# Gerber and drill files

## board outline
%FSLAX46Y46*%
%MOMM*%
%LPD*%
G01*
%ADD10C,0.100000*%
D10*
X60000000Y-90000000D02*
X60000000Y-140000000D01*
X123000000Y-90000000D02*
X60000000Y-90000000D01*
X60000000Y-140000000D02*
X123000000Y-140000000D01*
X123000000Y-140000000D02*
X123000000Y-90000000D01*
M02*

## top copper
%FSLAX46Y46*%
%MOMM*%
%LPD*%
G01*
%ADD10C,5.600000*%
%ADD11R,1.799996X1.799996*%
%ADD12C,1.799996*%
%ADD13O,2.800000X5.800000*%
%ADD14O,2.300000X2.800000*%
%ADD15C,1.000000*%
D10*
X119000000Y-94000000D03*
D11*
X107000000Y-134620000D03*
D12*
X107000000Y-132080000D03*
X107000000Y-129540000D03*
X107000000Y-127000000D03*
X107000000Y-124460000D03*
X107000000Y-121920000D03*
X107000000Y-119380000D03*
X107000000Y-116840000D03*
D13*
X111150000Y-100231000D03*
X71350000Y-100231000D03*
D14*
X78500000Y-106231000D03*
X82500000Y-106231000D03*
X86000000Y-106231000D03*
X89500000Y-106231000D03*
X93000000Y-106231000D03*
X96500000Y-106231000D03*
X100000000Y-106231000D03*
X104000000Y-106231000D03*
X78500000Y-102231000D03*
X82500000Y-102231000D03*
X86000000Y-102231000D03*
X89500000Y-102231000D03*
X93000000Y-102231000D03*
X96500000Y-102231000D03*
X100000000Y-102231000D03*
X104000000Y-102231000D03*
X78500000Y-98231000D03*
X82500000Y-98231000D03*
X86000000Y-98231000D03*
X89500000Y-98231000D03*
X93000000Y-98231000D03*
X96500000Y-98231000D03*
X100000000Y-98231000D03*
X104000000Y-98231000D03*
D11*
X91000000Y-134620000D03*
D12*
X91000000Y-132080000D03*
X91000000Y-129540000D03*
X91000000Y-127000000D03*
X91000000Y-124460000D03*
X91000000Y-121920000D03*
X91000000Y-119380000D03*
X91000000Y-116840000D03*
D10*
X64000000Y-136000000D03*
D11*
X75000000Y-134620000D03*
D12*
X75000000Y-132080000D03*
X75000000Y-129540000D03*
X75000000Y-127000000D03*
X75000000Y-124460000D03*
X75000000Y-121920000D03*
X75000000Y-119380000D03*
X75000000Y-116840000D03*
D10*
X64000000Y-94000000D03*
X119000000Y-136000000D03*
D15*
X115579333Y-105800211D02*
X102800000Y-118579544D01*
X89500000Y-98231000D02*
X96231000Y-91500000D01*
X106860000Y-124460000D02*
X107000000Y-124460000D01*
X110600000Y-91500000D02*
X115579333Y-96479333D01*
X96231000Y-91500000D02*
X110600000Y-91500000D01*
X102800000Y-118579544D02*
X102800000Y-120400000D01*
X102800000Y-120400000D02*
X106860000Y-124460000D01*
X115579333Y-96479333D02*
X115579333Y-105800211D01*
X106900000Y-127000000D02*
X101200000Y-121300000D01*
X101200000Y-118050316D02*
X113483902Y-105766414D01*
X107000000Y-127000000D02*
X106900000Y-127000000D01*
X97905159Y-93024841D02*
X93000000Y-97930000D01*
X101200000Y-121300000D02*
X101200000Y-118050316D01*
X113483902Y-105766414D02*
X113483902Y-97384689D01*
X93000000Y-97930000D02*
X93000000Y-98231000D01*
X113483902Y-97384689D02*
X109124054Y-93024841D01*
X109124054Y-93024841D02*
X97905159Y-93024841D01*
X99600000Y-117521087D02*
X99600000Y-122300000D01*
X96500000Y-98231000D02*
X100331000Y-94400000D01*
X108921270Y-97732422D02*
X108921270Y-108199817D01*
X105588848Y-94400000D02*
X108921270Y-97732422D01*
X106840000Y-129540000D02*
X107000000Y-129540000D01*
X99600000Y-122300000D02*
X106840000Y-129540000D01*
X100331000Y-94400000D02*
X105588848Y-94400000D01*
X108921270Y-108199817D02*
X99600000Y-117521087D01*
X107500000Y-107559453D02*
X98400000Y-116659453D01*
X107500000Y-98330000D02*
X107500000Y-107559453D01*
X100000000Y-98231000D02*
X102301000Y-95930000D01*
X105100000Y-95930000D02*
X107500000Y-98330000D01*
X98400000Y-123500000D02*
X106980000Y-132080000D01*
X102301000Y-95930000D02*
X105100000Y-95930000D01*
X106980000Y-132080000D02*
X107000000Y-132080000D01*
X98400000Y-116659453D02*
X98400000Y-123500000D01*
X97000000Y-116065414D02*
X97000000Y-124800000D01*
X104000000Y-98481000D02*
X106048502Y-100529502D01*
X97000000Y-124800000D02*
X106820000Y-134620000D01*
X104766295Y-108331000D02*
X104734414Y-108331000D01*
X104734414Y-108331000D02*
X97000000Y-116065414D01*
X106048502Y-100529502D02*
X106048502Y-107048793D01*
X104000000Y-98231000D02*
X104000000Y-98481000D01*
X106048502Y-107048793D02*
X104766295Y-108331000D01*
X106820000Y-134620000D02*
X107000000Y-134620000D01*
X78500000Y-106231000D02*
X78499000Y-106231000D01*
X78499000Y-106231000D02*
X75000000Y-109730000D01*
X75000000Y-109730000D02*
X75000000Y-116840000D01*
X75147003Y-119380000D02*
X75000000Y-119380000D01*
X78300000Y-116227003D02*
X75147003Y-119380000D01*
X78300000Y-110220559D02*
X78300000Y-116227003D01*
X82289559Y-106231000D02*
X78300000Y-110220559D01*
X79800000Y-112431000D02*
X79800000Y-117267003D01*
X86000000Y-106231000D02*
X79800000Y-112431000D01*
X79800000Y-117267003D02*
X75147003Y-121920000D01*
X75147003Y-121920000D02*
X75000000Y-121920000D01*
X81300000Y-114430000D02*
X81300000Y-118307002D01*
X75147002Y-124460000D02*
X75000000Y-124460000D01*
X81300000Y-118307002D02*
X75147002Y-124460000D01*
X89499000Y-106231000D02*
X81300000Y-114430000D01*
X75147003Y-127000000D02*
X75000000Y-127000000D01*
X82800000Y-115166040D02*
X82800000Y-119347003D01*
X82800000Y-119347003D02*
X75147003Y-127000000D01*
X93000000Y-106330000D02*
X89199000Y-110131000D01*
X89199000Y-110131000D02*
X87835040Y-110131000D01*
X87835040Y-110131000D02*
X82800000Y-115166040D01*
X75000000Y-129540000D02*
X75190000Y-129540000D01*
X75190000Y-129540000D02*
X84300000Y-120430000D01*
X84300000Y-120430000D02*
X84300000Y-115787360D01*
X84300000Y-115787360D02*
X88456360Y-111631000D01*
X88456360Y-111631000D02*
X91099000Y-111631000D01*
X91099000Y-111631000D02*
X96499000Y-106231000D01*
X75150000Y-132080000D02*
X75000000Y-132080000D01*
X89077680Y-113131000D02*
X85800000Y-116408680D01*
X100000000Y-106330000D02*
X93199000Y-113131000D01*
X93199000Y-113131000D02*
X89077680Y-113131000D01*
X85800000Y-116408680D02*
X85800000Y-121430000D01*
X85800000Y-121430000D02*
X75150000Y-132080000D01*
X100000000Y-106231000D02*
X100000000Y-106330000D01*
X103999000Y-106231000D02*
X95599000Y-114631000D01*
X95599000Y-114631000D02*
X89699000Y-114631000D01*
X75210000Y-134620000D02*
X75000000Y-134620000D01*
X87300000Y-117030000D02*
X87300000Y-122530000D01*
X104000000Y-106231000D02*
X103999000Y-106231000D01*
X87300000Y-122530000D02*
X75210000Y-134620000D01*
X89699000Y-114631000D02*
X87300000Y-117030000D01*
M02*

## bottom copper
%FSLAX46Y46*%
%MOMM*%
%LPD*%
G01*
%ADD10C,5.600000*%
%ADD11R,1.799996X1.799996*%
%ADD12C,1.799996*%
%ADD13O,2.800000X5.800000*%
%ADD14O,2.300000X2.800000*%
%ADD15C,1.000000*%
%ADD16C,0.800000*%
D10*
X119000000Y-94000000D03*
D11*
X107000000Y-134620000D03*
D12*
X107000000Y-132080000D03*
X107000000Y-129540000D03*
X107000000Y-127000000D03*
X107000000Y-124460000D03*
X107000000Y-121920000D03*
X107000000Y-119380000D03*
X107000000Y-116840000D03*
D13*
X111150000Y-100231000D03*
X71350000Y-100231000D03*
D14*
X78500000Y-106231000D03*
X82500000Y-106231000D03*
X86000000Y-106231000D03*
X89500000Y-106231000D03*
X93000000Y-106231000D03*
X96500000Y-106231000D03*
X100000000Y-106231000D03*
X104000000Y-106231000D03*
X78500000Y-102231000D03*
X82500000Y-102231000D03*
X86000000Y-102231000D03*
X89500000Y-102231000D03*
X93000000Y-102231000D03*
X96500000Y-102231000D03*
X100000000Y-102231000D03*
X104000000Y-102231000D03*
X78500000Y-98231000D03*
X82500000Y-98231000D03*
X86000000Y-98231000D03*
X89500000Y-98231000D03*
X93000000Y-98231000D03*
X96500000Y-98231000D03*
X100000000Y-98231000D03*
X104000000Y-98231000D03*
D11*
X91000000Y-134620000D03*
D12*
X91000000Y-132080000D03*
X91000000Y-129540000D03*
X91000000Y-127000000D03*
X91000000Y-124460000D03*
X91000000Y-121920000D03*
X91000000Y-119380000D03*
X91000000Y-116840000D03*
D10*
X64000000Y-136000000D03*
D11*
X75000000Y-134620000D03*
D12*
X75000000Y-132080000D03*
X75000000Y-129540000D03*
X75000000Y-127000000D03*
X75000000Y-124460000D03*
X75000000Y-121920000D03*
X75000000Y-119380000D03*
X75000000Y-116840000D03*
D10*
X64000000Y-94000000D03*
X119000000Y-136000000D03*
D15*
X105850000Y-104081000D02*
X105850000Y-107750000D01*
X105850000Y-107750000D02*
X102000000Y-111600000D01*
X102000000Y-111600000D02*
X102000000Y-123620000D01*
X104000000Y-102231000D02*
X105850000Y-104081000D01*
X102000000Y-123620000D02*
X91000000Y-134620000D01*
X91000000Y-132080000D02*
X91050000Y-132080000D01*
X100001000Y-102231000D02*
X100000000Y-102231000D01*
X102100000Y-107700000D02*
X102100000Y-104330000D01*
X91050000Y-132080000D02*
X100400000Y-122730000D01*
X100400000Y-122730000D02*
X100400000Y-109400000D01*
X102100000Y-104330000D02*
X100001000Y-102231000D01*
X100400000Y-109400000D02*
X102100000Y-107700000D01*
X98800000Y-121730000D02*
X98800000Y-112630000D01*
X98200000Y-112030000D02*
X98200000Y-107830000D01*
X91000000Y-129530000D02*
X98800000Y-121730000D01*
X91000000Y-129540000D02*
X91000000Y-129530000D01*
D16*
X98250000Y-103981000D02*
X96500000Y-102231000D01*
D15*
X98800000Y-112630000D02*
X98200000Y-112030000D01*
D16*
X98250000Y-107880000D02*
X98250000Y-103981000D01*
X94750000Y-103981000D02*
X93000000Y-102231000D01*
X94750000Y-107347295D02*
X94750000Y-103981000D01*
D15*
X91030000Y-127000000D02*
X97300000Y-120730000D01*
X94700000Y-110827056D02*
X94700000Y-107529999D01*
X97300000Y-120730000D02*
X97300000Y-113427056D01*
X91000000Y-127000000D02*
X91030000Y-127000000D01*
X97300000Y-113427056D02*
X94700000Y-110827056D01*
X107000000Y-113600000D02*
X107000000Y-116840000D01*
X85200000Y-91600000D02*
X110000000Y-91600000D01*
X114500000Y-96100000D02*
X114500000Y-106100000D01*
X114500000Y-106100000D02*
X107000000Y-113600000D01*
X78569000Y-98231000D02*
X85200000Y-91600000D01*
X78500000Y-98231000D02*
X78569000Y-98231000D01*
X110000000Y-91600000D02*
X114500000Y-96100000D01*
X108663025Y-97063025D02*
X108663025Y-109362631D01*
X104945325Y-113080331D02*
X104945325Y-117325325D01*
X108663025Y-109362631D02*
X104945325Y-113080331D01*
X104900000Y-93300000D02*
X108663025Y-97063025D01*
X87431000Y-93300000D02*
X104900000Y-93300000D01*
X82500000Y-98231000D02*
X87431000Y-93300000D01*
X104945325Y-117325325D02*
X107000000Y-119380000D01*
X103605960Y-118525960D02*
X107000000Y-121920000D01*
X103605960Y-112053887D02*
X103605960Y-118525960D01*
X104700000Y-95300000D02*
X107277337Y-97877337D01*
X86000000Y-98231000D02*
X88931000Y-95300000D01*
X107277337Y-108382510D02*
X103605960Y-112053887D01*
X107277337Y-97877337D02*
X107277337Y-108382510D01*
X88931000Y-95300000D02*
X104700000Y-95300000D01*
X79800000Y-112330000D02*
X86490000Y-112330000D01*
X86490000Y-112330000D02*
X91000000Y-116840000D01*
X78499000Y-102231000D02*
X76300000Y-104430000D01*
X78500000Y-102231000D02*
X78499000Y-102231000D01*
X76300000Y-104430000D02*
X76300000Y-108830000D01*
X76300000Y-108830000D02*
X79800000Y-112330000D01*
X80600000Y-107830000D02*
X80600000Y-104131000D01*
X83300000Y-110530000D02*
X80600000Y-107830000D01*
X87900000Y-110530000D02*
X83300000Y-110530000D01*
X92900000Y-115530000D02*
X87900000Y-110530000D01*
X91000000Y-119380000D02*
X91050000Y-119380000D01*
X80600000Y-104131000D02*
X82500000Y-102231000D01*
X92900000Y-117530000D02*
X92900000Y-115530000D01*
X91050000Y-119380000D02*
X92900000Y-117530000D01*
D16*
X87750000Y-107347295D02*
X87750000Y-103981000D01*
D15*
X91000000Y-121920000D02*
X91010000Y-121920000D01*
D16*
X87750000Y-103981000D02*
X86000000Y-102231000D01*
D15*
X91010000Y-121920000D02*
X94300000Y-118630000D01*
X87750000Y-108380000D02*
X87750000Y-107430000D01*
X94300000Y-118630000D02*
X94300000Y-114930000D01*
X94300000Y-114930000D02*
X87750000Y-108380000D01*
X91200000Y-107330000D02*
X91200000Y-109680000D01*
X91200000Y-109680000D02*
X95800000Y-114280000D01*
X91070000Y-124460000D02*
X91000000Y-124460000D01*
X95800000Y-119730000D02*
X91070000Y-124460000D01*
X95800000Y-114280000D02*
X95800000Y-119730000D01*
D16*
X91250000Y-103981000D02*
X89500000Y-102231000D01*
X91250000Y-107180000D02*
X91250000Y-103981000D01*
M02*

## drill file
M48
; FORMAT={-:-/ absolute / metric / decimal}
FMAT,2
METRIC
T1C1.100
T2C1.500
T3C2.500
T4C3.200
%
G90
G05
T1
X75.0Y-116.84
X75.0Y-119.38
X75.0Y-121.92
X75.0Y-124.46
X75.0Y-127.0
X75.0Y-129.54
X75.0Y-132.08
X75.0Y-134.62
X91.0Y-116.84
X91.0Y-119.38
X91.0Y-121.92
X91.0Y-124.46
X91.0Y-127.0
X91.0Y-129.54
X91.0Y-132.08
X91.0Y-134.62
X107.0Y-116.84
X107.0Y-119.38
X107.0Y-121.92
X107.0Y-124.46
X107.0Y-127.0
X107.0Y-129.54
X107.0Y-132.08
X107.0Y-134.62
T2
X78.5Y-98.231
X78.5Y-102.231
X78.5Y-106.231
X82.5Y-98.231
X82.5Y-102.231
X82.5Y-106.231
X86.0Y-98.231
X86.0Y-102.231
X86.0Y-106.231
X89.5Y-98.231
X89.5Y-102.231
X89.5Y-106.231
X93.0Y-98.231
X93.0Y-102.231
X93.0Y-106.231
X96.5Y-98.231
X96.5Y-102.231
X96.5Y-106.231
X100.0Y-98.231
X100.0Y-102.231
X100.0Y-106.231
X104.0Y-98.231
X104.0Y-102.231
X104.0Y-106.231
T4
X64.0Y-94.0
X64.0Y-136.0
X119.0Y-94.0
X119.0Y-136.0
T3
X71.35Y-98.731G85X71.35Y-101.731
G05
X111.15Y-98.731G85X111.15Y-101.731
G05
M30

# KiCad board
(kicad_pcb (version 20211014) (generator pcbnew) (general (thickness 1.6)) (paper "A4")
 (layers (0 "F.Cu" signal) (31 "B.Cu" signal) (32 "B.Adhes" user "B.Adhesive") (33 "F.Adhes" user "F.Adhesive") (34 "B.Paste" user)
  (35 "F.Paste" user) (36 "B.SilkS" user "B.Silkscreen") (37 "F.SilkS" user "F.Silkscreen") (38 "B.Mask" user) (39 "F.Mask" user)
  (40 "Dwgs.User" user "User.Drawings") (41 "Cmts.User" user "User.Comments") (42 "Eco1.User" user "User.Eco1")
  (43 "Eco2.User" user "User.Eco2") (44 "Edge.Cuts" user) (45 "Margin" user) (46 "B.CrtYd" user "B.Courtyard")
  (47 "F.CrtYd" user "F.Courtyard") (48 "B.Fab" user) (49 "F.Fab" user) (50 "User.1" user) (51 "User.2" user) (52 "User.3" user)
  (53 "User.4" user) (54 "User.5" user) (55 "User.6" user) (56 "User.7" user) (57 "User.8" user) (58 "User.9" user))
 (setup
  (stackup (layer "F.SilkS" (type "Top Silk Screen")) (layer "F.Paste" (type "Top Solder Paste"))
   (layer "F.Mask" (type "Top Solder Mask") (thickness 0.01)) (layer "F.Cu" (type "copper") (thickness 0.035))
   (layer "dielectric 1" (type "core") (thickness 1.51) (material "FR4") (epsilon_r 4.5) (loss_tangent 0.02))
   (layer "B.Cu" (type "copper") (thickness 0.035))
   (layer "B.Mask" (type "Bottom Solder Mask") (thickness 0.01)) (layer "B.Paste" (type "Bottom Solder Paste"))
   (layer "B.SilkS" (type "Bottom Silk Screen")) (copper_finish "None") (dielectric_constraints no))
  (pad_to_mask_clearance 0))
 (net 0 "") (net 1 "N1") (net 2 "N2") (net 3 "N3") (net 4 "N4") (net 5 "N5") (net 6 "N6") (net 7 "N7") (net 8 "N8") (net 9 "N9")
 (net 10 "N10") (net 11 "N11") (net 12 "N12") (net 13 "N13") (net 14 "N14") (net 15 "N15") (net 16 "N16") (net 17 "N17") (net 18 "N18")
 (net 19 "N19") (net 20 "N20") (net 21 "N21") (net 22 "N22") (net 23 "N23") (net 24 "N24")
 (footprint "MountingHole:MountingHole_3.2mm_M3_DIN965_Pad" (layer "F.Cu") (at 119 94 180)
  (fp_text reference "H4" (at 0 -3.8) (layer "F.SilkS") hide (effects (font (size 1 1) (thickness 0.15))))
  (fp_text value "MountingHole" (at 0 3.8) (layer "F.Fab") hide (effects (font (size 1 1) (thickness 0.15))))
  (pad "1" thru_hole circle locked (at 0 0 180) (size 5.6 5.6) (drill 3.2) (layers *.Cu *.Mask)))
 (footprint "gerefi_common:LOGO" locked (layer "F.Cu") (at 67.36 115.1)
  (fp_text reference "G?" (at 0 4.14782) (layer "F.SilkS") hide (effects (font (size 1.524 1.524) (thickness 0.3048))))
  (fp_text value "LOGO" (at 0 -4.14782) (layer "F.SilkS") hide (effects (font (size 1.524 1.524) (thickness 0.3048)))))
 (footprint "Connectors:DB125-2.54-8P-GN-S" (layer "F.Cu") (at 107 125.73 90)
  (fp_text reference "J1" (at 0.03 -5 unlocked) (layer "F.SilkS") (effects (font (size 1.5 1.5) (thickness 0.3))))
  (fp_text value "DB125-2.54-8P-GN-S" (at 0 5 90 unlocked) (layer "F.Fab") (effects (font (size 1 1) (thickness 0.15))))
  (pad "1" thru_hole rect (at -8.89 0 90) (size 1.799996 1.799996) (drill 1.100023) (layers *.Cu *.Mask) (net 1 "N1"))
  (pad "2" thru_hole circle (at -6.35 0 90) (size 1.799996 1.799996) (drill 1.100023) (layers *.Cu *.Mask) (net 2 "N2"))
  (pad "3" thru_hole circle (at -3.81 0 90) (size 1.799996 1.799996) (drill 1.100023) (layers *.Cu *.Mask) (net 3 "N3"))
  (pad "4" thru_hole circle (at -1.27 0 90) (size 1.799996 1.799996) (drill 1.100023) (layers *.Cu *.Mask) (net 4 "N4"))
  (pad "5" thru_hole circle (at 1.27 0 90) (size 1.799996 1.799996) (drill 1.100023) (layers *.Cu *.Mask) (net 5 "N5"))
  (pad "6" thru_hole circle (at 3.81 0 90) (size 1.799996 1.799996) (drill 1.100023) (layers *.Cu *.Mask) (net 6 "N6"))
  (pad "7" thru_hole circle (at 6.35 0 90) (size 1.799996 1.799996) (drill 1.100023) (layers *.Cu *.Mask) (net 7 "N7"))
  (pad "8" thru_hole circle (at 8.89 0 90) (size 1.799996 1.799996) (drill 1.100023) (layers *.Cu *.Mask) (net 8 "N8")))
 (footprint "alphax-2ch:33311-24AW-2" (layer "F.Cu") (at 78.5 106.231)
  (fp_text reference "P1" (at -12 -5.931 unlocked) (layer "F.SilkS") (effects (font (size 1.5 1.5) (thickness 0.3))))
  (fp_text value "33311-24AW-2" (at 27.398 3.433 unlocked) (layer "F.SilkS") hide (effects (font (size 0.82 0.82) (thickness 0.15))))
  (pad "" thru_hole oval locked (at 32.65 -6 270) (size 5.8 2.8) (drill oval 5.5 2.5) (layers *.Cu *.Mask) (solder_mask_margin 0.05))
  (pad "" thru_hole oval locked (at -7.15 -6 270) (size 5.8 2.8) (drill oval 5.5 2.5) (layers *.Cu *.Mask) (solder_mask_margin 0.05))
  (pad "1" thru_hole oval locked (at 0 0 270) (size 2.8 2.3) (drill 1.5) (layers *.Cu *.Mask) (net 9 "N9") (solder_mask_margin 0.05))
  (pad "2" thru_hole oval locked (at 4 0 270) (size 2.8 2.3) (drill 1.5) (layers *.Cu *.Mask) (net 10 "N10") (solder_mask_margin 0.05))
  (pad "3" thru_hole oval locked (at 7.5 0 270) (size 2.8 2.3) (drill 1.5) (layers *.Cu *.Mask) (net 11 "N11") (solder_mask_margin 0.05))
  (pad "4" thru_hole oval locked (at 11 0 270) (size 2.8 2.3) (drill 1.5) (layers *.Cu *.Mask) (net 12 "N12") (solder_mask_margin 0.05))
  (pad "5" thru_hole oval locked (at 14.5 0 270) (size 2.8 2.3) (drill 1.5) (layers *.Cu *.Mask) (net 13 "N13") (solder_mask_margin 0.05))
  (pad "6" thru_hole oval locked (at 18 0 270) (size 2.8 2.3) (drill 1.5) (layers *.Cu *.Mask) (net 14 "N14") (solder_mask_margin 0.05))
  (pad "7" thru_hole oval locked (at 21.5 0 270) (size 2.8 2.3) (drill 1.5) (layers *.Cu *.Mask) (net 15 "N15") (solder_mask_margin 0.05))
  (pad "8" thru_hole oval locked (at 25.5 0 270) (size 2.8 2.3) (drill 1.5) (layers *.Cu *.Mask) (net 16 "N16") (solder_mask_margin 0.05))
  (pad "9" thru_hole oval locked (at 0 -4 270) (size 2.8 2.3) (drill 1.5) (layers *.Cu *.Mask) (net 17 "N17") (solder_mask_margin 0.05))
  (pad "10" thru_hole oval locked (at 4 -4 270) (size 2.8 2.3) (drill 1.5) (layers *.Cu *.Mask) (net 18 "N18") (solder_mask_margin 0.05))
  (pad "11" thru_hole oval locked (at 7.5 -4 270) (size 2.8 2.3) (drill 1.5) (layers *.Cu *.Mask) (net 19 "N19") (solder_mask_margin 0.05))
  (pad "12" thru_hole oval locked (at 11 -4 270) (size 2.8 2.3) (drill 1.5) (layers *.Cu *.Mask) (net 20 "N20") (solder_mask_margin 0.05))
  (pad "13" thru_hole oval locked (at 14.5 -4 270) (size 2.8 2.3) (drill 1.5) (layers *.Cu *.Mask) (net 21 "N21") (solder_mask_margin 0.05))
  (pad "14" thru_hole oval locked (at 18 -4 270) (size 2.8 2.3) (drill 1.5) (layers *.Cu *.Mask) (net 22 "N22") (solder_mask_margin 0.05))
  (pad "15" thru_hole oval locked (at 21.5 -4 270) (size 2.8 2.3) (drill 1.5) (layers *.Cu *.Mask) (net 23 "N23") (solder_mask_margin 0.05))
  (pad "16" thru_hole oval locked (at 25.5 -4 270) (size 2.8 2.3) (drill 1.5) (layers *.Cu *.Mask) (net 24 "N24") (solder_mask_margin 0.05))
  (pad "17" thru_hole oval locked (at 0 -8 270) (size 2.8 2.3) (drill 1.5) (layers *.Cu *.Mask) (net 8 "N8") (solder_mask_margin 0.05))
  (pad "18" thru_hole oval locked (at 4 -8 270) (size 2.8 2.3) (drill 1.5) (layers *.Cu *.Mask) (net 7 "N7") (solder_mask_margin 0.05))
  (pad "19" thru_hole oval locked (at 7.5 -8 270) (size 2.8 2.3) (drill 1.5) (layers *.Cu *.Mask) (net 6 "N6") (solder_mask_margin 0.05))
  (pad "20" thru_hole oval locked (at 11 -8 270) (size 2.8 2.3) (drill 1.5) (layers *.Cu *.Mask) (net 5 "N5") (solder_mask_margin 0.05))
  (pad "21" thru_hole oval locked (at 14.5 -8 270) (size 2.8 2.3) (drill 1.5) (layers *.Cu *.Mask) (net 4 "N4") (solder_mask_margin 0.05))
  (pad "22" thru_hole oval locked (at 18 -8 270) (size 2.8 2.3) (drill 1.5) (layers *.Cu *.Mask) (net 3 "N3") (solder_mask_margin 0.05))
  (pad "23" thru_hole oval locked (at 21.5 -8 270) (size 2.8 2.3) (drill 1.5) (layers *.Cu *.Mask) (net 2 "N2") (solder_mask_margin 0.05))
  (pad "24" thru_hole oval locked (at 25.5 -8 270) (size 2.8 2.3) (drill 1.5) (layers *.Cu *.Mask) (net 1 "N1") (solder_mask_margin 0.05)))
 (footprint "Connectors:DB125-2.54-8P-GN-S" (layer "F.Cu") (at 91 125.73 90)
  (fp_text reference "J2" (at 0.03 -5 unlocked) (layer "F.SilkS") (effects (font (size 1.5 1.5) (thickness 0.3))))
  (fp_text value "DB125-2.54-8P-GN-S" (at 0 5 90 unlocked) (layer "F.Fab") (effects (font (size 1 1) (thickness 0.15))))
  (pad "1" thru_hole rect (at -8.89 0 90) (size 1.799996 1.799996) (drill 1.100023) (layers *.Cu *.Mask) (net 24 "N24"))
  (pad "2" thru_hole circle (at -6.35 0 90) (size 1.799996 1.799996) (drill 1.100023) (layers *.Cu *.Mask) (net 23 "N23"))
  (pad "3" thru_hole circle (at -3.81 0 90) (size 1.799996 1.799996) (drill 1.100023) (layers *.Cu *.Mask) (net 22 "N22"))
  (pad "4" thru_hole circle (at -1.27 0 90) (size 1.799996 1.799996) (drill 1.100023) (layers *.Cu *.Mask) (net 21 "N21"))
  (pad "5" thru_hole circle (at 1.27 0 90) (size 1.799996 1.799996) (drill 1.100023) (layers *.Cu *.Mask) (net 20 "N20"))
  (pad "6" thru_hole circle (at 3.81 0 90) (size 1.799996 1.799996) (drill 1.100023) (layers *.Cu *.Mask) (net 19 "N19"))
  (pad "7" thru_hole circle (at 6.35 0 90) (size 1.799996 1.799996) (drill 1.100023) (layers *.Cu *.Mask) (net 18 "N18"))
  (pad "8" thru_hole circle (at 8.89 0 90) (size 1.799996 1.799996) (drill 1.100023) (layers *.Cu *.Mask) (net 17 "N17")))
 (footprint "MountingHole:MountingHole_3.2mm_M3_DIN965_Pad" (layer "F.Cu") (at 64 136 180)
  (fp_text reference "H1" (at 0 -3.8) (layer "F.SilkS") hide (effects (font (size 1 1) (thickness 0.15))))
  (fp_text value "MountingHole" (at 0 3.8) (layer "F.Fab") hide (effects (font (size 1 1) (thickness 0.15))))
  (pad "1" thru_hole circle locked (at 0 0 180) (size 5.6 5.6) (drill 3.2) (layers *.Cu *.Mask)))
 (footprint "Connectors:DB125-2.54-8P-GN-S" (layer "F.Cu") (at 75 125.73 90)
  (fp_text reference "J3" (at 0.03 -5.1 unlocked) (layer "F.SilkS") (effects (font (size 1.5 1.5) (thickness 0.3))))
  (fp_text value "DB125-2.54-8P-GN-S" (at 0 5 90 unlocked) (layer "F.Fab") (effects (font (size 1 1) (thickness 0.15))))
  (pad "1" thru_hole rect (at -8.89 0 90) (size 1.799996 1.799996) (drill 1.100023) (layers *.Cu *.Mask) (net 16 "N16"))
  (pad "2" thru_hole circle (at -6.35 0 90) (size 1.799996 1.799996) (drill 1.100023) (layers *.Cu *.Mask) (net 15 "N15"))
  (pad "3" thru_hole circle (at -3.81 0 90) (size 1.799996 1.799996) (drill 1.100023) (layers *.Cu *.Mask) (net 14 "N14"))
  (pad "4" thru_hole circle (at -1.27 0 90) (size 1.799996 1.799996) (drill 1.100023) (layers *.Cu *.Mask) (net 13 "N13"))
  (pad "5" thru_hole circle (at 1.27 0 90) (size 1.799996 1.799996) (drill 1.100023) (layers *.Cu *.Mask) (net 12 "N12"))
  (pad "6" thru_hole circle (at 3.81 0 90) (size 1.799996 1.799996) (drill 1.100023) (layers *.Cu *.Mask) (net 11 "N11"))
  (pad "7" thru_hole circle (at 6.35 0 90) (size 1.799996 1.799996) (drill 1.100023) (layers *.Cu *.Mask) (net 10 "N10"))
  (pad "8" thru_hole circle (at 8.89 0 90) (size 1.799996 1.799996) (drill 1.100023) (layers *.Cu *.Mask) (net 9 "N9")))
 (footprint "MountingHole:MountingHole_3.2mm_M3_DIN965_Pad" (layer "F.Cu") (at 64 94 180)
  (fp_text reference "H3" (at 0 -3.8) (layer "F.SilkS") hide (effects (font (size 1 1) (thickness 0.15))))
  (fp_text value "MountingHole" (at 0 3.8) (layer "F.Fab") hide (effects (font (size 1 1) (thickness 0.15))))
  (pad "1" thru_hole circle locked (at 0 0 180) (size 5.6 5.6) (drill 3.2) (layers *.Cu *.Mask)))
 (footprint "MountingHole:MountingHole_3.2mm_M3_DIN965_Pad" (layer "F.Cu") (at 119 136 180)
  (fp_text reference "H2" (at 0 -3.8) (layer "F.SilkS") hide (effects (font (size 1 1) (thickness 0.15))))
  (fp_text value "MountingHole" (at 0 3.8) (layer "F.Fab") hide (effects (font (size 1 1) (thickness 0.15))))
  (pad "1" thru_hole circle locked (at 0 0 180) (size 5.6 5.6) (drill 3.2) (layers *.Cu *.Mask)))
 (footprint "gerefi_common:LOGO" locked (layer "B.Cu") (at 114.934286 115.2 180)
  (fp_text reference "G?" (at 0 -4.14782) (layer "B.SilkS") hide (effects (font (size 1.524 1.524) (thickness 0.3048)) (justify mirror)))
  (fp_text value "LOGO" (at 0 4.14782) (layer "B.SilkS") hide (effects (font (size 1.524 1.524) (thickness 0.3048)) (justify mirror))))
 (gr_line (start 60 90) (end 60 140) (layer "Edge.Cuts") (width 0.1))
 (gr_line (start 123 90) (end 60 90) (layer "Edge.Cuts") (width 0.1))
 (gr_line (start 60 140) (end 123 140) (layer "Edge.Cuts") (width 0.1))
 (gr_line (start 123 140) (end 123 90) (layer "Edge.Cuts") (width 0.1))
 (segment (start 105.85 104.081) (end 105.85 107.75) (width 1) (layer "B.Cu") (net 24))
 (segment (start 105.85 107.75) (end 102 111.6) (width 1) (layer "B.Cu") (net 24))
 (segment (start 102 111.6) (end 102 123.62) (width 1) (layer "B.Cu") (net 24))
 (segment (start 104 102.231) (end 105.85 104.081) (width 1) (layer "B.Cu") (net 24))
 (segment (start 102 123.62) (end 91 134.62) (width 1) (layer "B.Cu") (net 24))
 (segment (start 91 132.08) (end 91.05 132.08) (width 1) (layer "B.Cu") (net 23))
 (segment (start 100.001 102.231) (end 100 102.231) (width 1) (layer "B.Cu") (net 23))
 (segment (start 102.1 107.7) (end 102.1 104.33) (width 1) (layer "B.Cu") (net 23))
 (segment (start 91.05 132.08) (end 100.4 122.73) (width 1) (layer "B.Cu") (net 23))
 (segment (start 100.4 122.73) (end 100.4 109.4) (width 1) (layer "B.Cu") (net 23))
 (segment (start 102.1 104.33) (end 100.001 102.231) (width 1) (layer "B.Cu") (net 23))
 (segment (start 100.4 109.4) (end 102.1 107.7) (width 1) (layer "B.Cu") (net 23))
 (segment (start 98.8 121.73) (end 98.8 112.63) (width 1) (layer "B.Cu") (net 22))
 (segment (start 98.2 112.03) (end 98.2 107.83) (width 1) (layer "B.Cu") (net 22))
 (segment (start 91 129.53) (end 98.8 121.73) (width 1) (layer "B.Cu") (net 22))
 (segment (start 91 129.54) (end 91 129.53) (width 1) (layer "B.Cu") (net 22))
 (segment (start 98.25 103.981) (end 96.5 102.231) (width 0.8) (layer "B.Cu") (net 22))
 (segment (start 98.8 112.63) (end 98.2 112.03) (width 1) (layer "B.Cu") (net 22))
 (segment (start 98.25 107.88) (end 98.25 103.981) (width 0.8) (layer "B.Cu") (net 22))
 (segment (start 94.75 103.981) (end 93 102.231) (width 0.8) (layer "B.Cu") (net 21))
 (segment (start 94.75 107.347295) (end 94.75 103.981) (width 0.8) (layer "B.Cu") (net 21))
 (segment (start 91.03 127) (end 97.3 120.73) (width 1) (layer "B.Cu") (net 21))
 (segment (start 94.7 110.827056) (end 94.7 107.529999) (width 1) (layer "B.Cu") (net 21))
 (segment (start 97.3 120.73) (end 97.3 113.427056) (width 1) (layer "B.Cu") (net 21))
 (segment (start 91 127) (end 91.03 127) (width 1) (layer "B.Cu") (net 21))
 (segment (start 97.3 113.427056) (end 94.7 110.827056) (width 1) (layer "B.Cu") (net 21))
 (segment (start 107 113.6) (end 107 116.84) (width 1) (layer "B.Cu") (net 8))
 (segment (start 85.2 91.6) (end 110 91.6) (width 1) (layer "B.Cu") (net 8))
 (segment (start 114.5 96.1) (end 114.5 106.1) (width 1) (layer "B.Cu") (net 8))
 (segment (start 114.5 106.1) (end 107 113.6) (width 1) (layer "B.Cu") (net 8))
 (segment (start 78.569 98.231) (end 85.2 91.6) (width 1) (layer "B.Cu") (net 8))
 (segment (start 78.5 98.231) (end 78.569 98.231) (width 1) (layer "B.Cu") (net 8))
 (segment (start 110 91.6) (end 114.5 96.1) (width 1) (layer "B.Cu") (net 8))
 (segment (start 108.663025 97.063025) (end 108.663025 109.362631) (width 1) (layer "B.Cu") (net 7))
 (segment (start 104.945325 113.080331) (end 104.945325 117.325325) (width 1) (layer "B.Cu") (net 7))
 (segment (start 108.663025 109.362631) (end 104.945325 113.080331) (width 1) (layer "B.Cu") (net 7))
 (segment (start 104.9 93.3) (end 108.663025 97.063025) (width 1) (layer "B.Cu") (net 7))
 (segment (start 87.431 93.3) (end 104.9 93.3) (width 1) (layer "B.Cu") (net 7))
 (segment (start 82.5 98.231) (end 87.431 93.3) (width 1) (layer "B.Cu") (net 7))
 (segment (start 104.945325 117.325325) (end 107 119.38) (width 1) (layer "B.Cu") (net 7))
 (segment (start 103.60596 118.52596) (end 107 121.92) (width 1) (layer "B.Cu") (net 6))
 (segment (start 103.60596 112.053887) (end 103.60596 118.52596) (width 1) (layer "B.Cu") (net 6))
 (segment (start 104.7 95.3) (end 107.277337 97.877337) (width 1) (layer "B.Cu") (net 6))
 (segment (start 86 98.231) (end 88.931 95.3) (width 1) (layer "B.Cu") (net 6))
 (segment (start 107.277337 108.38251) (end 103.60596 112.053887) (width 1) (layer "B.Cu") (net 6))
 (segment (start 107.277337 97.877337) (end 107.277337 108.38251) (width 1) (layer "B.Cu") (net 6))
 (segment (start 88.931 95.3) (end 104.7 95.3) (width 1) (layer "B.Cu") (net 6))
 (segment (start 115.579333 105.800211) (end 102.8 118.579544) (width 1) (layer "F.Cu") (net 5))
 (segment (start 89.5 98.231) (end 96.231 91.5) (width 1) (layer "F.Cu") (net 5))
 (segment (start 106.86 124.46) (end 107 124.46) (width 1) (layer "F.Cu") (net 5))
 (segment (start 110.6 91.5) (end 115.579333 96.479333) (width 1) (layer "F.Cu") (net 5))
 (segment (start 96.231 91.5) (end 110.6 91.5) (width 1) (layer "F.Cu") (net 5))
 (segment (start 102.8 118.579544) (end 102.8 120.4) (width 1) (layer "F.Cu") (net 5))
 (segment (start 102.8 120.4) (end 106.86 124.46) (width 1) (layer "F.Cu") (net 5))
 (segment (start 115.579333 96.479333) (end 115.579333 105.800211) (width 1) (layer "F.Cu") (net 5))
 (segment (start 106.9 127) (end 101.2 121.3) (width 1) (layer "F.Cu") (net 4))
 (segment (start 101.2 118.050316) (end 113.483902 105.766414) (width 1) (layer "F.Cu") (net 4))
 (segment (start 107 127) (end 106.9 127) (width 1) (layer "F.Cu") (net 4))
 (segment (start 97.905159 93.024841) (end 93 97.93) (width 1) (layer "F.Cu") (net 4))
 (segment (start 101.2 121.3) (end 101.2 118.050316) (width 1) (layer "F.Cu") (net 4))
 (segment (start 113.483902 105.766414) (end 113.483902 97.384689) (width 1) (layer "F.Cu") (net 4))
 (segment (start 93 97.93) (end 93 98.231) (width 1) (layer "F.Cu") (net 4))
 (segment (start 113.483902 97.384689) (end 109.124054 93.024841) (width 1) (layer "F.Cu") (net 4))
 (segment (start 109.124054 93.024841) (end 97.905159 93.024841) (width 1) (layer "F.Cu") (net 4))
 (segment (start 99.6 117.521087) (end 99.6 122.3) (width 1) (layer "F.Cu") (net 3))
 (segment (start 96.5 98.231) (end 100.331 94.4) (width 1) (layer "F.Cu") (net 3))
 (segment (start 108.92127 97.732422) (end 108.92127 108.199817) (width 1) (layer "F.Cu") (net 3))
 (segment (start 105.588848 94.4) (end 108.92127 97.732422) (width 1) (layer "F.Cu") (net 3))
 (segment (start 106.84 129.54) (end 107 129.54) (width 1) (layer "F.Cu") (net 3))
 (segment (start 99.6 122.3) (end 106.84 129.54) (width 1) (layer "F.Cu") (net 3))
 (segment (start 100.331 94.4) (end 105.588848 94.4) (width 1) (layer "F.Cu") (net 3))
 (segment (start 108.92127 108.199817) (end 99.6 117.521087) (width 1) (layer "F.Cu") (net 3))
 (segment (start 107.5 107.559453) (end 98.4 116.659453) (width 1) (layer "F.Cu") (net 2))
 (segment (start 107.5 98.33) (end 107.5 107.559453) (width 1) (layer "F.Cu") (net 2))
 (segment (start 100 98.231) (end 102.301 95.93) (width 1) (layer "F.Cu") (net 2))
 (segment (start 105.1 95.93) (end 107.5 98.33) (width 1) (layer "F.Cu") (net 2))
 (segment (start 98.4 123.5) (end 106.98 132.08) (width 1) (layer "F.Cu") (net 2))
 (segment (start 102.301 95.93) (end 105.1 95.93) (width 1) (layer "F.Cu") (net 2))
 (segment (start 106.98 132.08) (end 107 132.08) (width 1) (layer "F.Cu") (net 2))
 (segment (start 98.4 116.659453) (end 98.4 123.5) (width 1) (layer "F.Cu") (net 2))
 (segment (start 97 116.065414) (end 97 124.8) (width 1) (layer "F.Cu") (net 1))
 (segment (start 104 98.481) (end 106.048502 100.529502) (width 1) (layer "F.Cu") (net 1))
 (segment (start 97 124.8) (end 106.82 134.62) (width 1) (layer "F.Cu") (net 1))
 (segment (start 104.766295 108.331) (end 104.734414 108.331) (width 1) (layer "F.Cu") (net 1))
 (segment (start 104.734414 108.331) (end 97 116.065414) (width 1) (layer "F.Cu") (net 1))
 (segment (start 106.048502 100.529502) (end 106.048502 107.048793) (width 1) (layer "F.Cu") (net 1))
 (segment (start 104 98.231) (end 104 98.481) (width 1) (layer "F.Cu") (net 1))
 (segment (start 106.048502 107.048793) (end 104.766295 108.331) (width 1) (layer "F.Cu") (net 1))
 (segment (start 106.82 134.62) (end 107 134.62) (width 1) (layer "F.Cu") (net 1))
 (segment (start 79.8 112.33) (end 86.49 112.33) (width 1) (layer "B.Cu") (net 17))
 (segment (start 86.49 112.33) (end 91 116.84) (width 1) (layer "B.Cu") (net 17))
 (segment (start 78.499 102.231) (end 76.3 104.43) (width 1) (layer "B.Cu") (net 17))
 (segment (start 78.5 102.231) (end 78.499 102.231) (width 1) (layer "B.Cu") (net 17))
 (segment (start 76.3 104.43) (end 76.3 108.83) (width 1) (layer "B.Cu") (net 17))
 (segment (start 76.3 108.83) (end 79.8 112.33) (width 1) (layer "B.Cu") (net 17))
 (segment (start 80.6 107.83) (end 80.6 104.131) (width 1) (layer "B.Cu") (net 18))
 (segment (start 83.3 110.53) (end 80.6 107.83) (width 1) (layer "B.Cu") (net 18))
 (segment (start 87.9 110.53) (end 83.3 110.53) (width 1) (layer "B.Cu") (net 18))
 (segment (start 92.9 115.53) (end 87.9 110.53) (width 1) (layer "B.Cu") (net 18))
 (segment (start 91 119.38) (end 91.05 119.38) (width 1) (layer "B.Cu") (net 18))
 (segment (start 80.6 104.131) (end 82.5 102.231) (width 1) (layer "B.Cu") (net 18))
 (segment (start 92.9 117.53) (end 92.9 115.53) (width 1) (layer "B.Cu") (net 18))
 (segment (start 91.05 119.38) (end 92.9 117.53) (width 1) (layer "B.Cu") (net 18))
 (segment (start 87.75 107.347295) (end 87.75 103.981) (width 0.8) (layer "B.Cu") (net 19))
 (segment (start 91 121.92) (end 91.01 121.92) (width 1) (layer "B.Cu") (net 19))
 (segment (start 87.75 103.981) (end 86 102.231) (width 0.8) (layer "B.Cu") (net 19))
 (segment (start 91.01 121.92) (end 94.3 118.63) (width 1) (layer "B.Cu") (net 19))
 (segment (start 87.75 108.38) (end 87.75 107.43) (width 1) (layer "B.Cu") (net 19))
 (segment (start 94.3 118.63) (end 94.3 114.93) (width 1) (layer "B.Cu") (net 19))
 (segment (start 94.3 114.93) (end 87.75 108.38) (width 1) (layer "B.Cu") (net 19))
 (segment (start 91.2 107.33) (end 91.2 109.68) (width 1) (layer "B.Cu") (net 20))
 (segment (start 91.2 109.68) (end 95.8 114.28) (width 1) (layer "B.Cu") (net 20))
 (segment (start 91.07 124.46) (end 91 124.46) (width 1) (layer "B.Cu") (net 20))
 (segment (start 95.8 119.73) (end 91.07 124.46) (width 1) (layer "B.Cu") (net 20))
 (segment (start 95.8 114.28) (end 95.8 119.73) (width 1) (layer "B.Cu") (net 20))
 (segment (start 91.25 103.981) (end 89.5 102.231) (width 0.8) (layer "B.Cu") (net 20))
 (segment (start 91.25 107.18) (end 91.25 103.981) (width 0.8) (layer "B.Cu") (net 20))
 (segment (start 78.5 106.231) (end 78.499 106.231) (width 1) (layer "F.Cu") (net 9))
 (segment (start 78.499 106.231) (end 75 109.73) (width 1) (layer "F.Cu") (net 9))
 (segment (start 75 109.73) (end 75 116.84) (width 1) (layer "F.Cu") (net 9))
 (segment (start 75.147003 119.38) (end 75 119.38) (width 1) (layer "F.Cu") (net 10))
 (segment (start 78.3 116.227003) (end 75.147003 119.38) (width 1) (layer "F.Cu") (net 10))
 (segment (start 78.3 110.220559) (end 78.3 116.227003) (width 1) (layer "F.Cu") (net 10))
 (segment (start 82.289559 106.231) (end 78.3 110.220559) (width 1) (layer "F.Cu") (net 10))
 (segment (start 79.8 112.431) (end 79.8 117.267003) (width 1) (layer "F.Cu") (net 11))
 (segment (start 86 106.231) (end 79.8 112.431) (width 1) (layer "F.Cu") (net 11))
 (segment (start 79.8 117.267003) (end 75.147003 121.92) (width 1) (layer "F.Cu") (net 11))
 (segment (start 75.147003 121.92) (end 75 121.92) (width 1) (layer "F.Cu") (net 11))
 (segment (start 81.3 114.43) (end 81.3 118.307002) (width 1) (layer "F.Cu") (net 12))
 (segment (start 75.147002 124.46) (end 75 124.46) (width 1) (layer "F.Cu") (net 12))
 (segment (start 81.3 118.307002) (end 75.147002 124.46) (width 1) (layer "F.Cu") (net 12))
 (segment (start 89.499 106.231) (end 81.3 114.43) (width 1) (layer "F.Cu") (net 12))
 (segment (start 75.147003 127) (end 75 127) (width 1) (layer "F.Cu") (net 13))
 (segment (start 82.8 115.16604) (end 82.8 119.347003) (width 1) (layer "F.Cu") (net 13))
 (segment (start 82.8 119.347003) (end 75.147003 127) (width 1) (layer "F.Cu") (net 13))
 (segment (start 93 106.33) (end 89.199 110.131) (width 1) (layer "F.Cu") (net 13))
 (segment (start 89.199 110.131) (end 87.83504 110.131) (width 1) (layer "F.Cu") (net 13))
 (segment (start 87.83504 110.131) (end 82.8 115.16604) (width 1) (layer "F.Cu") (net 13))
 (segment (start 75 129.54) (end 75.19 129.54) (width 1) (layer "F.Cu") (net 14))
 (segment (start 75.19 129.54) (end 84.3 120.43) (width 1) (layer "F.Cu") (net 14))
 (segment (start 84.3 120.43) (end 84.3 115.78736) (width 1) (layer "F.Cu") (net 14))
 (segment (start 84.3 115.78736) (end 88.45636 111.631) (width 1) (layer "F.Cu") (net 14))
 (segment (start 88.45636 111.631) (end 91.099 111.631) (width 1) (layer "F.Cu") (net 14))
 (segment (start 91.099 111.631) (end 96.499 106.231) (width 1) (layer "F.Cu") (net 14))
 (segment (start 75.15 132.08) (end 75 132.08) (width 1) (layer "F.Cu") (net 15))
 (segment (start 89.07768 113.131) (end 85.8 116.40868) (width 1) (layer "F.Cu") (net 15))
 (segment (start 100 106.33) (end 93.199 113.131) (width 1) (layer "F.Cu") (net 15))
 (segment (start 93.199 113.131) (end 89.07768 113.131) (width 1) (layer "F.Cu") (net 15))
 (segment (start 85.8 116.40868) (end 85.8 121.43) (width 1) (layer "F.Cu") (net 15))
 (segment (start 85.8 121.43) (end 75.15 132.08) (width 1) (layer "F.Cu") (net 15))
 (segment (start 100 106.231) (end 100 106.33) (width 1) (layer "F.Cu") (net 15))
 (segment (start 103.999 106.231) (end 95.599 114.631) (width 1) (layer "F.Cu") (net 16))
 (segment (start 95.599 114.631) (end 89.699 114.631) (width 1) (layer "F.Cu") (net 16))
 (segment (start 75.21 134.62) (end 75 134.62) (width 1) (layer "F.Cu") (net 16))
 (segment (start 87.3 117.03) (end 87.3 122.53) (width 1) (layer "F.Cu") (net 16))
 (segment (start 104 106.231) (end 103.999 106.231) (width 1) (layer "F.Cu") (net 16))
 (segment (start 87.3 122.53) (end 75.21 134.62) (width 1) (layer "F.Cu") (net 16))
 (segment (start 89.699 114.631) (end 87.3 117.03) (width 1) (layer "F.Cu") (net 16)))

